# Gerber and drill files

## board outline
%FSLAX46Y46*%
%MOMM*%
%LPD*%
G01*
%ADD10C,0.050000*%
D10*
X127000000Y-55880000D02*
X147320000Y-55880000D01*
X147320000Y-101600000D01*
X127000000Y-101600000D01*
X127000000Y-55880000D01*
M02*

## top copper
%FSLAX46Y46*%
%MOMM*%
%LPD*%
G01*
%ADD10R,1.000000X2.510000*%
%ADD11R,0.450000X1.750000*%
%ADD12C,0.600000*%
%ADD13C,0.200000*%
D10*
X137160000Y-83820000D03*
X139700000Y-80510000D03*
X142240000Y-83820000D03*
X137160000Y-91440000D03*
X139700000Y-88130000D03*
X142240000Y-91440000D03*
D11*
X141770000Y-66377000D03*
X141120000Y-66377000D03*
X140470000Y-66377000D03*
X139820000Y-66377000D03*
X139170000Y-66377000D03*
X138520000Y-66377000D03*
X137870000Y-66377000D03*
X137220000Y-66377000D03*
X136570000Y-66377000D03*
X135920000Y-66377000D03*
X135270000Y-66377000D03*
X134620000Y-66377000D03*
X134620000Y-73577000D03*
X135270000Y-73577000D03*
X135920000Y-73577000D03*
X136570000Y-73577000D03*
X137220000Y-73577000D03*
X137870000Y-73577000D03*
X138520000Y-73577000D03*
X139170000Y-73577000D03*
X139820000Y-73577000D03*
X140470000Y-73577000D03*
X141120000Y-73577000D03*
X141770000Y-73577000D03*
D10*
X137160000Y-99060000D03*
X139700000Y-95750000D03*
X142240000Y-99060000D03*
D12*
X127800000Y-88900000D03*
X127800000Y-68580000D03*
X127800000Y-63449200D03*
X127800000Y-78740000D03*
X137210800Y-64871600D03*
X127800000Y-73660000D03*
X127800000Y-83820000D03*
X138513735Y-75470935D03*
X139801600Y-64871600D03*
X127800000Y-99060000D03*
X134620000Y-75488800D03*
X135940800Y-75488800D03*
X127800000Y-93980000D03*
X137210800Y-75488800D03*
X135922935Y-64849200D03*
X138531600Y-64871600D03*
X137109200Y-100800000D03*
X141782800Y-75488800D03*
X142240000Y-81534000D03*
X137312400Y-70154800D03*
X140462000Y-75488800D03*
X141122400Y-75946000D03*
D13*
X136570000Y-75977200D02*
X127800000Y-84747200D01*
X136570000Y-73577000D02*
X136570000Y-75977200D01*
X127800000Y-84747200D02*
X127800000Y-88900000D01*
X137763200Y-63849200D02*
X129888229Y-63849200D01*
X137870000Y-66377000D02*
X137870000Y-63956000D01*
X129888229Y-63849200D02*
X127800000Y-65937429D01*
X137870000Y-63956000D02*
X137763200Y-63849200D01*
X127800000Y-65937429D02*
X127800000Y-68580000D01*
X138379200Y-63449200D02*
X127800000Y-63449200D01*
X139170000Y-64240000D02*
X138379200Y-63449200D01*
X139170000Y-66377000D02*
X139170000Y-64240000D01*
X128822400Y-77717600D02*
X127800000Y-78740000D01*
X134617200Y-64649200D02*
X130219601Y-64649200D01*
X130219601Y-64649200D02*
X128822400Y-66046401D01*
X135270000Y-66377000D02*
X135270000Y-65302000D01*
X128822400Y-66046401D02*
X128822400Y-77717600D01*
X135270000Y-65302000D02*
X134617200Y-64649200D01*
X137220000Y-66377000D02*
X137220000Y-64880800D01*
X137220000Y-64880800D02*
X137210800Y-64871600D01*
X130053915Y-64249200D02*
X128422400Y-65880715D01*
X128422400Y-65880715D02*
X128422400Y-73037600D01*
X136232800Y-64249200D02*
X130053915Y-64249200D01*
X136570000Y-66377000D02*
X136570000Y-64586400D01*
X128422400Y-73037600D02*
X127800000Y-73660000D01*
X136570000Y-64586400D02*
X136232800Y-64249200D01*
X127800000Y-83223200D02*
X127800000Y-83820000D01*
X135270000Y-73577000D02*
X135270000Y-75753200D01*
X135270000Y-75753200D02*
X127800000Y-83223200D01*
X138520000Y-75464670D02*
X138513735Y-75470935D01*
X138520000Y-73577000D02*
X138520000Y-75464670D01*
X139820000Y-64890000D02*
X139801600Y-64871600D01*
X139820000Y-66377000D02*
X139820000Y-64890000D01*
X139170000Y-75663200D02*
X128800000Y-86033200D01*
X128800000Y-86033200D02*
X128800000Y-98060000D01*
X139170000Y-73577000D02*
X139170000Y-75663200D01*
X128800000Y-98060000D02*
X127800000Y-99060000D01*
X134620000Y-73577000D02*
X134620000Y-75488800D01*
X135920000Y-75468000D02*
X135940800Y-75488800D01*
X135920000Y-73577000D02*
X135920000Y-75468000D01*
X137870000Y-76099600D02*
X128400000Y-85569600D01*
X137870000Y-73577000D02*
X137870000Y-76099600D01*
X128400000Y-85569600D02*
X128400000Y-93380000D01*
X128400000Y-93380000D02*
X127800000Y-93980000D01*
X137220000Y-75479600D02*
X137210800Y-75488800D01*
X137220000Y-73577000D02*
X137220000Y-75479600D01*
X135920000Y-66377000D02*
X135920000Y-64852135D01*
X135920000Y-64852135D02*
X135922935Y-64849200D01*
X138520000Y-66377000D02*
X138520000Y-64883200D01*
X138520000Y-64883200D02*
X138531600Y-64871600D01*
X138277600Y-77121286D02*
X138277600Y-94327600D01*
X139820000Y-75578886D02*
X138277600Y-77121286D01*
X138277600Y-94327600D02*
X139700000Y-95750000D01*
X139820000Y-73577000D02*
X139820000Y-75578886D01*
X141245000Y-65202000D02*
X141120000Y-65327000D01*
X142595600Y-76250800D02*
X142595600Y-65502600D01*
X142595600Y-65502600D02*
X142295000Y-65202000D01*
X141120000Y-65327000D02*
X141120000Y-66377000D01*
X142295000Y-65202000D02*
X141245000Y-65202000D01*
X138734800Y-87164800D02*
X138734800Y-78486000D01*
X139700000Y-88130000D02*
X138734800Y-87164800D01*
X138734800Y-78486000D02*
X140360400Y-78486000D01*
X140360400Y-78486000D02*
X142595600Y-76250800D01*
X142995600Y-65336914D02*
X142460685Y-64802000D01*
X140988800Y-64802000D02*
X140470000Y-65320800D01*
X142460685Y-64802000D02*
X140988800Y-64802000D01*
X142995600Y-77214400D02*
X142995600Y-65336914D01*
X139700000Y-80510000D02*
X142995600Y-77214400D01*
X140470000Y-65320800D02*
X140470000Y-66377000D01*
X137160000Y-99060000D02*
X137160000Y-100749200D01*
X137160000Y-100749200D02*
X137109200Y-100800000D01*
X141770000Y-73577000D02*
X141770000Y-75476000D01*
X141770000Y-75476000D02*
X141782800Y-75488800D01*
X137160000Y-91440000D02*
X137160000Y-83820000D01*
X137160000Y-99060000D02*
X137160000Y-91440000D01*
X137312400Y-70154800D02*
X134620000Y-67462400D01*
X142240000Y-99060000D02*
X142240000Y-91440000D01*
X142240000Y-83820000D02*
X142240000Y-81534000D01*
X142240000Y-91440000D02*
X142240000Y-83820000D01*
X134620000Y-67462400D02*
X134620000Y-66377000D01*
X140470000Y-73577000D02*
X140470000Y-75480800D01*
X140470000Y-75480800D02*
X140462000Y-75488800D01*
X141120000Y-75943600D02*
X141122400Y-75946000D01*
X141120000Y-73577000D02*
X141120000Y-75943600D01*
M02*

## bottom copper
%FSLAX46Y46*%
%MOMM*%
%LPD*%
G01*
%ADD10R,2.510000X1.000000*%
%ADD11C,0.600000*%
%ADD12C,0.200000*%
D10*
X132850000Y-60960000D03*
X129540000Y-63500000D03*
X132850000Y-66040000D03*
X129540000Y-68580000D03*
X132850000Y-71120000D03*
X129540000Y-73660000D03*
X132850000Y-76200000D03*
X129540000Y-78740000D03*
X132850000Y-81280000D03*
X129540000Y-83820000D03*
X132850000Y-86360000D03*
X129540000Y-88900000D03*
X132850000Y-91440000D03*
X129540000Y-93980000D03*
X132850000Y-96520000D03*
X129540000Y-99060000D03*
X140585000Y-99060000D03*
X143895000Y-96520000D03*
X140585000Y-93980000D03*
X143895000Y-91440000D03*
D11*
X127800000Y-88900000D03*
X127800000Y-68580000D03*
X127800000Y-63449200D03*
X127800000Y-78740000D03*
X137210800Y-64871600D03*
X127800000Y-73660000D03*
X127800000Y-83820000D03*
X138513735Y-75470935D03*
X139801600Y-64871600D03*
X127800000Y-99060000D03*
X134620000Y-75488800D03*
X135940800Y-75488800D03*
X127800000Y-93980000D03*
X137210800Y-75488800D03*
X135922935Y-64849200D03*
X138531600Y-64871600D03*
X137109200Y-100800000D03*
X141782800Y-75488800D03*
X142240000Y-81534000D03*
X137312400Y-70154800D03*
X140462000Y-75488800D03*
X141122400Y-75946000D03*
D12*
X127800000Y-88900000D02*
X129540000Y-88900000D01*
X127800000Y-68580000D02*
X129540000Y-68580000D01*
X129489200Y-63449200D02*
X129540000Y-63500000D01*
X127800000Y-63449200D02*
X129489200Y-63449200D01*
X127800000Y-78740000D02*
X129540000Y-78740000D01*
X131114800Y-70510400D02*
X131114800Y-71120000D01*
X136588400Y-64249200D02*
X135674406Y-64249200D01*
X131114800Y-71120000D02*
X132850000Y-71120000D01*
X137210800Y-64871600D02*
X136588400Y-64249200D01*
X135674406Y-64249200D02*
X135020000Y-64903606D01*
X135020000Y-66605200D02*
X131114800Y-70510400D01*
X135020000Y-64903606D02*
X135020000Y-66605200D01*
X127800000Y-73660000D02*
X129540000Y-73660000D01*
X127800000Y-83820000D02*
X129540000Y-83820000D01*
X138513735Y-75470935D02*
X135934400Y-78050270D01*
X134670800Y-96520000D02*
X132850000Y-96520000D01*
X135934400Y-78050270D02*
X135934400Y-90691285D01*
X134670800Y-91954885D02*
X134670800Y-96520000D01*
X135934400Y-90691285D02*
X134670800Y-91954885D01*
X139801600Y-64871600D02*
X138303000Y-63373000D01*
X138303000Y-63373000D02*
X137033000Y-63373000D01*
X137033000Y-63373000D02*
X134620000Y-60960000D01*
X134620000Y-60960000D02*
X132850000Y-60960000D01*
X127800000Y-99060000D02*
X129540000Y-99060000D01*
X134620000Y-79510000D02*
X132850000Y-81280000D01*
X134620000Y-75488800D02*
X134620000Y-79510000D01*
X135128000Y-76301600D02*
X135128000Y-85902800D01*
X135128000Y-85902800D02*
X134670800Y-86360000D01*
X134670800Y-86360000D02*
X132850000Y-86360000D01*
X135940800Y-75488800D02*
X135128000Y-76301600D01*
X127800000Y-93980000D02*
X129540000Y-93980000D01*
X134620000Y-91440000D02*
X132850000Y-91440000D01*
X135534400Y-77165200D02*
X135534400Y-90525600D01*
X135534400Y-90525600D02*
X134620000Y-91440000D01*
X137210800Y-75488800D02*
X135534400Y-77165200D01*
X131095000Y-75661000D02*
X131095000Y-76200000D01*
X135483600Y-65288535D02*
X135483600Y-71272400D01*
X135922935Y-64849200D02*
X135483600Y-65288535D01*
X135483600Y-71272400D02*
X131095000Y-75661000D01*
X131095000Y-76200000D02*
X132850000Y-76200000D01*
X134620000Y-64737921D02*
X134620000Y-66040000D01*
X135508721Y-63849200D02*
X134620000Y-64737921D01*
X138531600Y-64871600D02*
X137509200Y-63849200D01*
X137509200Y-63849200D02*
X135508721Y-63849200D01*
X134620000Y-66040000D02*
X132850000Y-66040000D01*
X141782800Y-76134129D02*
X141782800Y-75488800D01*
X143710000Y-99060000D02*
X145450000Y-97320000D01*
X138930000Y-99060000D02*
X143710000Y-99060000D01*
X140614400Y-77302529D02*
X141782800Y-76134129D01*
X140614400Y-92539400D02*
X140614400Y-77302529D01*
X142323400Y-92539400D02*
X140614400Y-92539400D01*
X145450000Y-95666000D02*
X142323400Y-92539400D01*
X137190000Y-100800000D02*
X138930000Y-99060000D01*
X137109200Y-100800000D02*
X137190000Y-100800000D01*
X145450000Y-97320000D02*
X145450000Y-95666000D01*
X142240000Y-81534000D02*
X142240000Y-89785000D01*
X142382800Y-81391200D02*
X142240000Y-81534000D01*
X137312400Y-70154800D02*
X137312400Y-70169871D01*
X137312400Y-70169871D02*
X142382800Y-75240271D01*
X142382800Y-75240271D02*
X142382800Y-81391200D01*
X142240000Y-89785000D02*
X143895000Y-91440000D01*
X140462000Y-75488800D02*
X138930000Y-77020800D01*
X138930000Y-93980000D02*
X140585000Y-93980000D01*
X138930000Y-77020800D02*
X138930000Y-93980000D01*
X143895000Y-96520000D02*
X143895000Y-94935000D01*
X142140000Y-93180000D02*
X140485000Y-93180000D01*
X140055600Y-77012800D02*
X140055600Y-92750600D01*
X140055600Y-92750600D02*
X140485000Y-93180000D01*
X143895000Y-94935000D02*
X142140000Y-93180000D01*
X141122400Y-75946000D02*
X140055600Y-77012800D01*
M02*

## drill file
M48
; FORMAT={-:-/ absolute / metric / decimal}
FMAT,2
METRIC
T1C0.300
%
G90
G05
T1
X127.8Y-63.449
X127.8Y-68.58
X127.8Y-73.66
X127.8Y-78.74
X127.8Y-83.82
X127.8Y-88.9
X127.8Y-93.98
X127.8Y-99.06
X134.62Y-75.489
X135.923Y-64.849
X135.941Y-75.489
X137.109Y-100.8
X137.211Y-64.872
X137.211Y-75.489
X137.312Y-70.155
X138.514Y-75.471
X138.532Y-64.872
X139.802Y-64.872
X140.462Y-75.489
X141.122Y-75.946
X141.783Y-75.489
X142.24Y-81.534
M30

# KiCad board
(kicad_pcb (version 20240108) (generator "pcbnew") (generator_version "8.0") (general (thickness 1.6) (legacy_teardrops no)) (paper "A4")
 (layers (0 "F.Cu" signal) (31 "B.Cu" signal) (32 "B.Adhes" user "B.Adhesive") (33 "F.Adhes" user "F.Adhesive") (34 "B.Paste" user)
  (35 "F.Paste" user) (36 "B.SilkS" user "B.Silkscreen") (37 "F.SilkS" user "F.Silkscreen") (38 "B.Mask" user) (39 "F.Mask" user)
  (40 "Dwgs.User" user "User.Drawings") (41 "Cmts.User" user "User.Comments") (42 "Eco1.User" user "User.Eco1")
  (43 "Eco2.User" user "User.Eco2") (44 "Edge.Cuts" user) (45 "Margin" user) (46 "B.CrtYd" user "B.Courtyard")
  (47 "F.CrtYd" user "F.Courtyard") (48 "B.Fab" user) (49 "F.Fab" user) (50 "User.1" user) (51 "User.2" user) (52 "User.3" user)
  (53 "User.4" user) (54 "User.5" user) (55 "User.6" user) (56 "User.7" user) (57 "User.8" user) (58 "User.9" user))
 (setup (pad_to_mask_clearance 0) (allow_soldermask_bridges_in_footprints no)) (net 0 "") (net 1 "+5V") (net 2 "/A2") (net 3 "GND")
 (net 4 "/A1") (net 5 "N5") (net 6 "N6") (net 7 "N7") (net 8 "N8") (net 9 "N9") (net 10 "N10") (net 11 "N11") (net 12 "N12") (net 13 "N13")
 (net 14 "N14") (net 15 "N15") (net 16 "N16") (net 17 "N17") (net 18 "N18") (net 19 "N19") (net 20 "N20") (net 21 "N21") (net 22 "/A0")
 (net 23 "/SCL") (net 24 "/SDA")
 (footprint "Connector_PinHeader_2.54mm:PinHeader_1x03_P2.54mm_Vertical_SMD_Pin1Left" (layer "F.Cu") (at 139.7 82.165 90)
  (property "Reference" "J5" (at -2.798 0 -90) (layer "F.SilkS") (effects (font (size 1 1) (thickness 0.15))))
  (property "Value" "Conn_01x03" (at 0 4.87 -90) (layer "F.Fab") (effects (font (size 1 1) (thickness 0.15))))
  (pad "1" smd rect (at -1.655 -2.54 90) (size 2.51 1) (layers "F.Cu" "F.Paste" "F.Mask") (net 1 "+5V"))
  (pad "2" smd rect (at 1.655 0 90) (size 2.51 1) (layers "F.Cu" "F.Paste" "F.Mask") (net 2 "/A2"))
  (pad "3" smd rect (at -1.655 2.54 90) (size 2.51 1) (layers "F.Cu" "F.Paste" "F.Mask") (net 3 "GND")))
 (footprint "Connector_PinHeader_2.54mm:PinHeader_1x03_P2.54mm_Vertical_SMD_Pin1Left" (layer "F.Cu") (at 139.7 89.785 90)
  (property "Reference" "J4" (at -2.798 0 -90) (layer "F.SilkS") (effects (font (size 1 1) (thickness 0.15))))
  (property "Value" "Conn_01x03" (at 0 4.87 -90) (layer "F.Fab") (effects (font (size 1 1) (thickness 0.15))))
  (pad "1" smd rect (at -1.655 -2.54 90) (size 2.51 1) (layers "F.Cu" "F.Paste" "F.Mask") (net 1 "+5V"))
  (pad "2" smd rect (at 1.655 0 90) (size 2.51 1) (layers "F.Cu" "F.Paste" "F.Mask") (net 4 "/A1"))
  (pad "3" smd rect (at -1.655 2.54 90) (size 2.51 1) (layers "F.Cu" "F.Paste" "F.Mask") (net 3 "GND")))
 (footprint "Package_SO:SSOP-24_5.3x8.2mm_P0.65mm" (layer "F.Cu") (at 138.195 69.977 -90)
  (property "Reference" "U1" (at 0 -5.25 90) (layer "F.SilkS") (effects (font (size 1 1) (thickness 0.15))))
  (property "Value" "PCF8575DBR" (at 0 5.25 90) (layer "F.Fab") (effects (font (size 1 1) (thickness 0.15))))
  (pad "1" smd rect (at -3.6 -3.575 270) (size 1.75 0.45) (layers "F.Cu" "F.Paste" "F.Mask") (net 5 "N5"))
  (pad "2" smd rect (at -3.6 -2.925 270) (size 1.75 0.45) (layers "F.Cu" "F.Paste" "F.Mask") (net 4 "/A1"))
  (pad "3" smd rect (at -3.6 -2.275 270) (size 1.75 0.45) (layers "F.Cu" "F.Paste" "F.Mask") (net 2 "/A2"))
  (pad "4" smd rect (at -3.6 -1.625 270) (size 1.75 0.45) (layers "F.Cu" "F.Paste" "F.Mask") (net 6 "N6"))
  (pad "5" smd rect (at -3.6 -0.975 270) (size 1.75 0.45) (layers "F.Cu" "F.Paste" "F.Mask") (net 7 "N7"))
  (pad "6" smd rect (at -3.6 -0.325 270) (size 1.75 0.45) (layers "F.Cu" "F.Paste" "F.Mask") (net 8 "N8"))
  (pad "7" smd rect (at -3.6 0.325 270) (size 1.75 0.45) (layers "F.Cu" "F.Paste" "F.Mask") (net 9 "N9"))
  (pad "8" smd rect (at -3.6 0.975 270) (size 1.75 0.45) (layers "F.Cu" "F.Paste" "F.Mask") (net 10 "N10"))
  (pad "9" smd rect (at -3.6 1.625 270) (size 1.75 0.45) (layers "F.Cu" "F.Paste" "F.Mask") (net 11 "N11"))
  (pad "10" smd rect (at -3.6 2.275 270) (size 1.75 0.45) (layers "F.Cu" "F.Paste" "F.Mask") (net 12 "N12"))
  (pad "11" smd rect (at -3.6 2.925 270) (size 1.75 0.45) (layers "F.Cu" "F.Paste" "F.Mask") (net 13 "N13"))
  (pad "12" smd rect (at -3.6 3.575 270) (size 1.75 0.45) (layers "F.Cu" "F.Paste" "F.Mask") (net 3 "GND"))
  (pad "13" smd rect (at 3.6 3.575 270) (size 1.75 0.45) (layers "F.Cu" "F.Paste" "F.Mask") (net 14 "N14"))
  (pad "14" smd rect (at 3.6 2.925 270) (size 1.75 0.45) (layers "F.Cu" "F.Paste" "F.Mask") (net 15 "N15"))
  (pad "15" smd rect (at 3.6 2.275 270) (size 1.75 0.45) (layers "F.Cu" "F.Paste" "F.Mask") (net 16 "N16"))
  (pad "16" smd rect (at 3.6 1.625 270) (size 1.75 0.45) (layers "F.Cu" "F.Paste" "F.Mask") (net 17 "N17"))
  (pad "17" smd rect (at 3.6 0.975 270) (size 1.75 0.45) (layers "F.Cu" "F.Paste" "F.Mask") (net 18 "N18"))
  (pad "18" smd rect (at 3.6 0.325 270) (size 1.75 0.45) (layers "F.Cu" "F.Paste" "F.Mask") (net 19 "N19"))
  (pad "19" smd rect (at 3.6 -0.325 270) (size 1.75 0.45) (layers "F.Cu" "F.Paste" "F.Mask") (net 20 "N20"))
  (pad "20" smd rect (at 3.6 -0.975 270) (size 1.75 0.45) (layers "F.Cu" "F.Paste" "F.Mask") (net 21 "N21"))
  (pad "21" smd rect (at 3.6 -1.625 270) (size 1.75 0.45) (layers "F.Cu" "F.Paste" "F.Mask") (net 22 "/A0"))
  (pad "22" smd rect (at 3.6 -2.275 270) (size 1.75 0.45) (layers "F.Cu" "F.Paste" "F.Mask") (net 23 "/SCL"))
  (pad "23" smd rect (at 3.6 -2.925 270) (size 1.75 0.45) (layers "F.Cu" "F.Paste" "F.Mask") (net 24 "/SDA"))
  (pad "24" smd rect (at 3.6 -3.575 270) (size 1.75 0.45) (layers "F.Cu" "F.Paste" "F.Mask") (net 1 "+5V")))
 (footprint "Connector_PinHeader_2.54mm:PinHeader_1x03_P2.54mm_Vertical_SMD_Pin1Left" (layer "F.Cu") (at 139.7 97.405 90)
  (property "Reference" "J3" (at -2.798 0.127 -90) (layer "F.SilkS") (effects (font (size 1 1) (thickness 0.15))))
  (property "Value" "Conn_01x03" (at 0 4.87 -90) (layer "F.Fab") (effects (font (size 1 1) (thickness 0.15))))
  (pad "1" smd rect (at -1.655 -2.54 90) (size 2.51 1) (layers "F.Cu" "F.Paste" "F.Mask") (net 1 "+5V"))
  (pad "2" smd rect (at 1.655 0 90) (size 2.51 1) (layers "F.Cu" "F.Paste" "F.Mask") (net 22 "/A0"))
  (pad "3" smd rect (at -1.655 2.54 90) (size 2.51 1) (layers "F.Cu" "F.Paste" "F.Mask") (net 3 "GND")))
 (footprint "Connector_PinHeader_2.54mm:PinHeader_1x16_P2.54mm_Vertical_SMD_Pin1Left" (layer "B.Cu") (at 131.195 80.01 180)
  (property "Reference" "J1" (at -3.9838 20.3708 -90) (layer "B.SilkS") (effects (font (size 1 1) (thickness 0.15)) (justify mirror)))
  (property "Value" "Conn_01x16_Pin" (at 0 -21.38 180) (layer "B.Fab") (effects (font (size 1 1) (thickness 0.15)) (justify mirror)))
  (pad "1" smd rect (at -1.655 19.05 180) (size 2.51 1) (layers "B.Cu" "B.Paste" "B.Mask") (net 6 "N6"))
  (pad "2" smd rect (at 1.655 16.51 180) (size 2.51 1) (layers "B.Cu" "B.Paste" "B.Mask") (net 7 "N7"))
  (pad "3" smd rect (at -1.655 13.97 180) (size 2.51 1) (layers "B.Cu" "B.Paste" "B.Mask") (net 8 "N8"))
  (pad "4" smd rect (at 1.655 11.43 180) (size 2.51 1) (layers "B.Cu" "B.Paste" "B.Mask") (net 9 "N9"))
  (pad "5" smd rect (at -1.655 8.89 180) (size 2.51 1) (layers "B.Cu" "B.Paste" "B.Mask") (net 10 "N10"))
  (pad "6" smd rect (at 1.655 6.35 180) (size 2.51 1) (layers "B.Cu" "B.Paste" "B.Mask") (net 11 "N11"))
  (pad "7" smd rect (at -1.655 3.81 180) (size 2.51 1) (layers "B.Cu" "B.Paste" "B.Mask") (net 12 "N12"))
  (pad "8" smd rect (at 1.655 1.27 180) (size 2.51 1) (layers "B.Cu" "B.Paste" "B.Mask") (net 13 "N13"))
  (pad "9" smd rect (at -1.655 -1.27 180) (size 2.51 1) (layers "B.Cu" "B.Paste" "B.Mask") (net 14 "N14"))
  (pad "10" smd rect (at 1.655 -3.81 180) (size 2.51 1) (layers "B.Cu" "B.Paste" "B.Mask") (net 15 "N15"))
  (pad "11" smd rect (at -1.655 -6.35 180) (size 2.51 1) (layers "B.Cu" "B.Paste" "B.Mask") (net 16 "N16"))
  (pad "12" smd rect (at 1.655 -8.89 180) (size 2.51 1) (layers "B.Cu" "B.Paste" "B.Mask") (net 17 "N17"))
  (pad "13" smd rect (at -1.655 -11.43 180) (size 2.51 1) (layers "B.Cu" "B.Paste" "B.Mask") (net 18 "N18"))
  (pad "14" smd rect (at 1.655 -13.97 180) (size 2.51 1) (layers "B.Cu" "B.Paste" "B.Mask") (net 19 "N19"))
  (pad "15" smd rect (at -1.655 -16.51 180) (size 2.51 1) (layers "B.Cu" "B.Paste" "B.Mask") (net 20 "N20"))
  (pad "16" smd rect (at 1.655 -19.05 180) (size 2.51 1) (layers "B.Cu" "B.Paste" "B.Mask") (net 21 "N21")))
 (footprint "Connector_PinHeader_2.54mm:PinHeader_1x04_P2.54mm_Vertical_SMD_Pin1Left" (layer "B.Cu") (at 142.24 95.25)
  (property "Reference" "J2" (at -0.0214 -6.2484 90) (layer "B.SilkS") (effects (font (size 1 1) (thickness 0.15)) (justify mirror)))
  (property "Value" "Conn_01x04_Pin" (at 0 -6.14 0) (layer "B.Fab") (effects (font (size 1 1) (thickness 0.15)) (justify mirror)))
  (pad "1" smd rect (at -1.655 3.81) (size 2.51 1) (layers "B.Cu" "B.Paste" "B.Mask") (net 1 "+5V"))
  (pad "2" smd rect (at 1.655 1.27) (size 2.51 1) (layers "B.Cu" "B.Paste" "B.Mask") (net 24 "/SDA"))
  (pad "3" smd rect (at -1.655 -1.27) (size 2.51 1) (layers "B.Cu" "B.Paste" "B.Mask") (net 23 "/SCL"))
  (pad "4" smd rect (at 1.655 -3.81) (size 2.51 1) (layers "B.Cu" "B.Paste" "B.Mask") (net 3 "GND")))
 (gr_rect (start 127 55.88) (end 147.32 101.6) (stroke (width 0.05) (type default)) (fill none) (layer "Edge.Cuts"))
 (segment (start 136.57 75.9772) (end 127.8 84.7472) (width 0.2) (layer "F.Cu") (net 17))
 (segment (start 136.57 73.577) (end 136.57 75.9772) (width 0.2) (layer "F.Cu") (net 17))
 (segment (start 127.8 84.7472) (end 127.8 88.9) (width 0.2) (layer "F.Cu") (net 17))
 (via (at 127.8 88.9) (size 0.6) (drill 0.3) (layers "F.Cu" "B.Cu") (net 17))
 (segment (start 127.8 88.9) (end 129.54 88.9) (width 0.2) (layer "B.Cu") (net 17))
 (segment (start 137.7632 63.8492) (end 129.888229 63.8492) (width 0.2) (layer "F.Cu") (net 9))
 (segment (start 137.87 66.377) (end 137.87 63.956) (width 0.2) (layer "F.Cu") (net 9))
 (segment (start 129.888229 63.8492) (end 127.8 65.937429) (width 0.2) (layer "F.Cu") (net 9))
 (segment (start 137.87 63.956) (end 137.7632 63.8492) (width 0.2) (layer "F.Cu") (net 9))
 (segment (start 127.8 65.937429) (end 127.8 68.58) (width 0.2) (layer "F.Cu") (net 9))
 (via (at 127.8 68.58) (size 0.6) (drill 0.3) (layers "F.Cu" "B.Cu") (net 9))
 (segment (start 127.8 68.58) (end 129.54 68.58) (width 0.2) (layer "B.Cu") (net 9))
 (segment (start 138.3792 63.4492) (end 127.8 63.4492) (width 0.2) (layer "F.Cu") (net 7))
 (segment (start 139.17 64.24) (end 138.3792 63.4492) (width 0.2) (layer "F.Cu") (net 7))
 (segment (start 139.17 66.377) (end 139.17 64.24) (width 0.2) (layer "F.Cu") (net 7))
 (via (at 127.8 63.4492) (size 0.6) (drill 0.3) (layers "F.Cu" "B.Cu") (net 7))
 (segment (start 129.4892 63.4492) (end 129.54 63.5) (width 0.2) (layer "B.Cu") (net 7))
 (segment (start 127.8 63.4492) (end 129.4892 63.4492) (width 0.2) (layer "B.Cu") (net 7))
 (segment (start 128.8224 77.7176) (end 127.8 78.74) (width 0.2) (layer "F.Cu") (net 13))
 (segment (start 134.6172 64.6492) (end 130.219601 64.6492) (width 0.2) (layer "F.Cu") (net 13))
 (segment (start 130.219601 64.6492) (end 128.8224 66.046401) (width 0.2) (layer "F.Cu") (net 13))
 (segment (start 135.27 66.377) (end 135.27 65.302) (width 0.2) (layer "F.Cu") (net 13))
 (segment (start 128.8224 66.046401) (end 128.8224 77.7176) (width 0.2) (layer "F.Cu") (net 13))
 (segment (start 135.27 65.302) (end 134.6172 64.6492) (width 0.2) (layer "F.Cu") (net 13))
 (via (at 127.8 78.74) (size 0.6) (drill 0.3) (layers "F.Cu" "B.Cu") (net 13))
 (segment (start 127.8 78.74) (end 129.54 78.74) (width 0.2) (layer "B.Cu") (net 13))
 (segment (start 137.22 66.377) (end 137.22 64.8808) (width 0.2) (layer "F.Cu") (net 10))
 (segment (start 137.22 64.8808) (end 137.2108 64.8716) (width 0.2) (layer "F.Cu") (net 10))
 (via (at 137.2108 64.8716) (size 0.6) (drill 0.3) (layers "F.Cu" "B.Cu") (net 10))
 (segment (start 131.1148 70.5104) (end 131.1148 71.12) (width 0.2) (layer "B.Cu") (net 10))
 (segment (start 136.5884 64.2492) (end 135.674406 64.2492) (width 0.2) (layer "B.Cu") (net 10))
 (segment (start 131.1148 71.12) (end 132.85 71.12) (width 0.2) (layer "B.Cu") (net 10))
 (segment (start 137.2108 64.8716) (end 136.5884 64.2492) (width 0.2) (layer "B.Cu") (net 10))
 (segment (start 135.674406 64.2492) (end 135.02 64.903606) (width 0.2) (layer "B.Cu") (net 10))
 (segment (start 135.02 66.6052) (end 131.1148 70.5104) (width 0.2) (layer "B.Cu") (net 10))
 (segment (start 135.02 64.903606) (end 135.02 66.6052) (width 0.2) (layer "B.Cu") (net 10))
 (segment (start 130.053915 64.2492) (end 128.4224 65.880715) (width 0.2) (layer "F.Cu") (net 11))
 (segment (start 128.4224 65.880715) (end 128.4224 73.0376) (width 0.2) (layer "F.Cu") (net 11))
 (segment (start 136.2328 64.2492) (end 130.053915 64.2492) (width 0.2) (layer "F.Cu") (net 11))
 (segment (start 136.57 66.377) (end 136.57 64.5864) (width 0.2) (layer "F.Cu") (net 11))
 (segment (start 128.4224 73.0376) (end 127.8 73.66) (width 0.2) (layer "F.Cu") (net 11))
 (segment (start 136.57 64.5864) (end 136.2328 64.2492) (width 0.2) (layer "F.Cu") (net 11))
 (via (at 127.8 73.66) (size 0.6) (drill 0.3) (layers "F.Cu" "B.Cu") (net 11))
 (segment (start 127.8 73.66) (end 129.54 73.66) (width 0.2) (layer "B.Cu") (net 11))
 (segment (start 127.8 83.2232) (end 127.8 83.82) (width 0.2) (layer "F.Cu") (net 15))
 (segment (start 135.27 73.577) (end 135.27 75.7532) (width 0.2) (layer "F.Cu") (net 15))
 (segment (start 135.27 75.7532) (end 127.8 83.2232) (width 0.2) (layer "F.Cu") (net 15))
 (via (at 127.8 83.82) (size 0.6) (drill 0.3) (layers "F.Cu" "B.Cu") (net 15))
 (segment (start 127.8 83.82) (end 129.54 83.82) (width 0.2) (layer "B.Cu") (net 15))
 (segment (start 138.52 75.46467) (end 138.513735 75.470935) (width 0.2) (layer "F.Cu") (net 20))
 (segment (start 138.52 73.577) (end 138.52 75.46467) (width 0.2) (layer "F.Cu") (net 20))
 (via (at 138.513735 75.470935) (size 0.6) (drill 0.3) (layers "F.Cu" "B.Cu") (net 20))
 (segment (start 138.513735 75.470935) (end 135.9344 78.05027) (width 0.2) (layer "B.Cu") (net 20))
 (segment (start 134.6708 96.52) (end 132.85 96.52) (width 0.2) (layer "B.Cu") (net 20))
 (segment (start 135.9344 78.05027) (end 135.9344 90.691285) (width 0.2) (layer "B.Cu") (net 20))
 (segment (start 134.6708 91.954885) (end 134.6708 96.52) (width 0.2) (layer "B.Cu") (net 20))
 (segment (start 135.9344 90.691285) (end 134.6708 91.954885) (width 0.2) (layer "B.Cu") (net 20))
 (segment (start 139.82 64.89) (end 139.8016 64.8716) (width 0.2) (layer "F.Cu") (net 6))
 (segment (start 139.82 66.377) (end 139.82 64.89) (width 0.2) (layer "F.Cu") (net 6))
 (via (at 139.8016 64.8716) (size 0.6) (drill 0.3) (layers "F.Cu" "B.Cu") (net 6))
 (segment (start 139.8016 64.8716) (end 138.303 63.373) (width 0.2) (layer "B.Cu") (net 6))
 (segment (start 138.303 63.373) (end 137.033 63.373) (width 0.2) (layer "B.Cu") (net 6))
 (segment (start 137.033 63.373) (end 134.62 60.96) (width 0.2) (layer "B.Cu") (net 6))
 (segment (start 134.62 60.96) (end 132.85 60.96) (width 0.2) (layer "B.Cu") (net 6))
 (segment (start 139.17 75.6632) (end 128.8 86.0332) (width 0.2) (layer "F.Cu") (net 21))
 (segment (start 128.8 86.0332) (end 128.8 98.06) (width 0.2) (layer "F.Cu") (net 21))
 (segment (start 139.17 73.577) (end 139.17 75.6632) (width 0.2) (layer "F.Cu") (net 21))
 (segment (start 128.8 98.06) (end 127.8 99.06) (width 0.2) (layer "F.Cu") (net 21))
 (via (at 127.8 99.06) (size 0.6) (drill 0.3) (layers "F.Cu" "B.Cu") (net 21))
 (segment (start 127.8 99.06) (end 129.54 99.06) (width 0.2) (layer "B.Cu") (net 21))
 (segment (start 134.62 73.577) (end 134.62 75.4888) (width 0.2) (layer "F.Cu") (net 14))
 (via (at 134.62 75.4888) (size 0.6) (drill 0.3) (layers "F.Cu" "B.Cu") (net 14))
 (segment (start 134.62 79.51) (end 132.85 81.28) (width 0.2) (layer "B.Cu") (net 14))
 (segment (start 134.62 75.4888) (end 134.62 79.51) (width 0.2) (layer "B.Cu") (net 14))
 (segment (start 135.92 75.468) (end 135.9408 75.4888) (width 0.2) (layer "F.Cu") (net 16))
 (segment (start 135.92 73.577) (end 135.92 75.468) (width 0.2) (layer "F.Cu") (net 16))
 (via (at 135.9408 75.4888) (size 0.6) (drill 0.3) (layers "F.Cu" "B.Cu") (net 16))
 (segment (start 135.128 76.3016) (end 135.128 85.9028) (width 0.2) (layer "B.Cu") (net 16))
 (segment (start 135.128 85.9028) (end 134.6708 86.36) (width 0.2) (layer "B.Cu") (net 16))
 (segment (start 134.6708 86.36) (end 132.85 86.36) (width 0.2) (layer "B.Cu") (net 16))
 (segment (start 135.9408 75.4888) (end 135.128 76.3016) (width 0.2) (layer "B.Cu") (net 16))
 (segment (start 137.87 76.0996) (end 128.4 85.5696) (width 0.2) (layer "F.Cu") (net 19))
 (segment (start 137.87 73.577) (end 137.87 76.0996) (width 0.2) (layer "F.Cu") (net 19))
 (segment (start 128.4 85.5696) (end 128.4 93.38) (width 0.2) (layer "F.Cu") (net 19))
 (segment (start 128.4 93.38) (end 127.8 93.98) (width 0.2) (layer "F.Cu") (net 19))
 (via (at 127.8 93.98) (size 0.6) (drill 0.3) (layers "F.Cu" "B.Cu") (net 19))
 (segment (start 127.8 93.98) (end 129.54 93.98) (width 0.2) (layer "B.Cu") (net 19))
 (segment (start 137.22 75.4796) (end 137.2108 75.4888) (width 0.2) (layer "F.Cu") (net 18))
 (segment (start 137.22 73.577) (end 137.22 75.4796) (width 0.2) (layer "F.Cu") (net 18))
 (via (at 137.2108 75.4888) (size 0.6) (drill 0.3) (layers "F.Cu" "B.Cu") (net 18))
 (segment (start 134.62 91.44) (end 132.85 91.44) (width 0.2) (layer "B.Cu") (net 18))
 (segment (start 135.5344 77.1652) (end 135.5344 90.5256) (width 0.2) (layer "B.Cu") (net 18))
 (segment (start 135.5344 90.5256) (end 134.62 91.44) (width 0.2) (layer "B.Cu") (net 18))
 (segment (start 137.2108 75.4888) (end 135.5344 77.1652) (width 0.2) (layer "B.Cu") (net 18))
 (segment (start 135.92 66.377) (end 135.92 64.852135) (width 0.2) (layer "F.Cu") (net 12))
 (segment (start 135.92 64.852135) (end 135.922935 64.8492) (width 0.2) (layer "F.Cu") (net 12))
 (via (at 135.922935 64.8492) (size 0.6) (drill 0.3) (layers "F.Cu" "B.Cu") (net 12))
 (segment (start 131.095 75.661) (end 131.095 76.2) (width 0.2) (layer "B.Cu") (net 12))
 (segment (start 135.4836 65.288535) (end 135.4836 71.2724) (width 0.2) (layer "B.Cu") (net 12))
 (segment (start 135.922935 64.8492) (end 135.4836 65.288535) (width 0.2) (layer "B.Cu") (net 12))
 (segment (start 135.4836 71.2724) (end 131.095 75.661) (width 0.2) (layer "B.Cu") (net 12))
 (segment (start 131.095 76.2) (end 132.85 76.2) (width 0.2) (layer "B.Cu") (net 12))
 (segment (start 138.52 66.377) (end 138.52 64.8832) (width 0.2) (layer "F.Cu") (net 8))
 (segment (start 138.52 64.8832) (end 138.5316 64.8716) (width 0.2) (layer "F.Cu") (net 8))
 (via (at 138.5316 64.8716) (size 0.6) (drill 0.3) (layers "F.Cu" "B.Cu") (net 8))
 (segment (start 134.62 64.737921) (end 134.62 66.04) (width 0.2) (layer "B.Cu") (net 8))
 (segment (start 135.508721 63.8492) (end 134.62 64.737921) (width 0.2) (layer "B.Cu") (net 8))
 (segment (start 138.5316 64.8716) (end 137.5092 63.8492) (width 0.2) (layer "B.Cu") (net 8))
 (segment (start 137.5092 63.8492) (end 135.508721 63.8492) (width 0.2) (layer "B.Cu") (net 8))
 (segment (start 134.62 66.04) (end 132.85 66.04) (width 0.2) (layer "B.Cu") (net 8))
 (segment (start 138.2776 77.121286) (end 138.2776 94.3276) (width 0.2) (layer "F.Cu") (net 22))
 (segment (start 139.82 75.578886) (end 138.2776 77.121286) (width 0.2) (layer "F.Cu") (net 22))
 (segment (start 138.2776 94.3276) (end 139.7 95.75) (width 0.2) (layer "F.Cu") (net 22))
 (segment (start 139.82 73.577) (end 139.82 75.578886) (width 0.2) (layer "F.Cu") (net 22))
 (segment (start 141.245 65.202) (end 141.12 65.327) (width 0.2) (layer "F.Cu") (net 4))
 (segment (start 142.5956 76.2508) (end 142.5956 65.5026) (width 0.2) (layer "F.Cu") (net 4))
 (segment (start 142.5956 65.5026) (end 142.295 65.202) (width 0.2) (layer "F.Cu") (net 4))
 (segment (start 141.12 65.327) (end 141.12 66.377) (width 0.2) (layer "F.Cu") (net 4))
 (segment (start 142.295 65.202) (end 141.245 65.202) (width 0.2) (layer "F.Cu") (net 4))
 (segment (start 138.7348 87.1648) (end 138.7348 78.486) (width 0.2) (layer "F.Cu") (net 4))
 (segment (start 139.7 88.13) (end 138.7348 87.1648) (width 0.2) (layer "F.Cu") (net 4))
 (segment (start 138.7348 78.486) (end 140.3604 78.486) (width 0.2) (layer "F.Cu") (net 4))
 (segment (start 140.3604 78.486) (end 142.5956 76.2508) (width 0.2) (layer "F.Cu") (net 4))
 (segment (start 142.9956 65.336914) (end 142.460685 64.802) (width 0.2) (layer "F.Cu") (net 2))
 (segment (start 140.9888 64.802) (end 140.47 65.3208) (width 0.2) (layer "F.Cu") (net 2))
 (segment (start 142.460685 64.802) (end 140.9888 64.802) (width 0.2) (layer "F.Cu") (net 2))
 (segment (start 142.9956 77.2144) (end 142.9956 65.336914) (width 0.2) (layer "F.Cu") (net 2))
 (segment (start 139.7 80.51) (end 142.9956 77.2144) (width 0.2) (layer "F.Cu") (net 2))
 (segment (start 140.47 65.3208) (end 140.47 66.377) (width 0.2) (layer "F.Cu") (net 2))
 (segment (start 137.16 99.06) (end 137.16 100.7492) (width 0.2) (layer "F.Cu") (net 1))
 (segment (start 137.16 100.7492) (end 137.1092 100.8) (width 0.2) (layer "F.Cu") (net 1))
 (segment (start 141.77 73.577) (end 141.77 75.476) (width 0.2) (layer "F.Cu") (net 1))
 (segment (start 141.77 75.476) (end 141.7828 75.4888) (width 0.2) (layer "F.Cu") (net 1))
 (segment (start 137.16 91.44) (end 137.16 83.82) (width 0.2) (layer "F.Cu") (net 1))
 (segment (start 137.16 99.06) (end 137.16 91.44) (width 0.2) (layer "F.Cu") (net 1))
 (via (at 137.1092 100.8) (size 0.6) (drill 0.3) (layers "F.Cu" "B.Cu") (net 1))
 (via (at 141.7828 75.4888) (size 0.6) (drill 0.3) (layers "F.Cu" "B.Cu") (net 1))
 (segment (start 141.7828 76.134129) (end 141.7828 75.4888) (width 0.2) (layer "B.Cu") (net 1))
 (segment (start 143.71 99.06) (end 145.45 97.32) (width 0.2) (layer "B.Cu") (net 1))
 (segment (start 138.93 99.06) (end 143.71 99.06) (width 0.2) (layer "B.Cu") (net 1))
 (segment (start 140.6144 77.302529) (end 141.7828 76.134129) (width 0.2) (layer "B.Cu") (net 1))
 (segment (start 140.6144 92.5394) (end 140.6144 77.302529) (width 0.2) (layer "B.Cu") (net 1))
 (segment (start 142.3234 92.5394) (end 140.6144 92.5394) (width 0.2) (layer "B.Cu") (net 1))
 (segment (start 145.45 95.666) (end 142.3234 92.5394) (width 0.2) (layer "B.Cu") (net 1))
 (segment (start 137.19 100.8) (end 138.93 99.06) (width 0.2) (layer "B.Cu") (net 1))
 (segment (start 137.1092 100.8) (end 137.19 100.8) (width 0.2) (layer "B.Cu") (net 1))
 (segment (start 145.45 97.32) (end 145.45 95.666) (width 0.2) (layer "B.Cu") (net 1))
 (segment (start 137.3124 70.1548) (end 134.62 67.4624) (width 0.2) (layer "F.Cu") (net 3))
 (segment (start 142.24 99.06) (end 142.24 91.44) (width 0.2) (layer "F.Cu") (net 3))
 (segment (start 142.24 83.82) (end 142.24 81.534) (width 0.2) (layer "F.Cu") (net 3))
 (segment (start 142.24 91.44) (end 142.24 83.82) (width 0.2) (layer "F.Cu") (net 3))
 (segment (start 134.62 67.4624) (end 134.62 66.377) (width 0.2) (layer "F.Cu") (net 3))
 (via (at 142.24 81.534) (size 0.6) (drill 0.3) (layers "F.Cu" "B.Cu") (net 3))
 (via (at 137.3124 70.1548) (size 0.6) (drill 0.3) (layers "F.Cu" "B.Cu") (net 3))
 (segment (start 142.24 81.534) (end 142.24 89.785) (width 0.2) (layer "B.Cu") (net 3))
 (segment (start 142.3828 81.3912) (end 142.24 81.534) (width 0.2) (layer "B.Cu") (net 3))
 (segment (start 137.3124 70.1548) (end 137.3124 70.169871) (width 0.2) (layer "B.Cu") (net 3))
 (segment (start 137.3124 70.169871) (end 142.3828 75.240271) (width 0.2) (layer "B.Cu") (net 3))
 (segment (start 142.3828 75.240271) (end 142.3828 81.3912) (width 0.2) (layer "B.Cu") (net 3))
 (segment (start 142.24 89.785) (end 143.895 91.44) (width 0.2) (layer "B.Cu") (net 3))
 (segment (start 140.47 73.577) (end 140.47 75.4808) (width 0.2) (layer "F.Cu") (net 23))
 (segment (start 140.47 75.4808) (end 140.462 75.4888) (width 0.2) (layer "F.Cu") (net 23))
 (via (at 140.462 75.4888) (size 0.6) (drill 0.3) (layers "F.Cu" "B.Cu") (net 23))
 (segment (start 140.462 75.4888) (end 138.93 77.0208) (width 0.2) (layer "B.Cu") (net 23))
 (segment (start 138.93 93.98) (end 140.585 93.98) (width 0.2) (layer "B.Cu") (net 23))
 (segment (start 138.93 77.0208) (end 138.93 93.98) (width 0.2) (layer "B.Cu") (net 23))
 (segment (start 141.12 75.9436) (end 141.1224 75.946) (width 0.2) (layer "F.Cu") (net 24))
 (segment (start 141.12 73.577) (end 141.12 75.9436) (width 0.2) (layer "F.Cu") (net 24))
 (via (at 141.1224 75.946) (size 0.6) (drill 0.3) (layers "F.Cu" "B.Cu") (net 24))
 (segment (start 143.895 96.52) (end 143.895 94.935) (width 0.2) (layer "B.Cu") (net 24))
 (segment (start 142.14 93.18) (end 140.485 93.18) (width 0.2) (layer "B.Cu") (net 24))
 (segment (start 140.0556 77.0128) (end 140.0556 92.7506) (width 0.2) (layer "B.Cu") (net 24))
 (segment (start 140.0556 92.7506) (end 140.485 93.18) (width 0.2) (layer "B.Cu") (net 24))
 (segment (start 143.895 94.935) (end 142.14 93.18) (width 0.2) (layer "B.Cu") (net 24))
 (segment (start 141.1224 75.946) (end 140.0556 77.0128) (width 0.2) (layer "B.Cu") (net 24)))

